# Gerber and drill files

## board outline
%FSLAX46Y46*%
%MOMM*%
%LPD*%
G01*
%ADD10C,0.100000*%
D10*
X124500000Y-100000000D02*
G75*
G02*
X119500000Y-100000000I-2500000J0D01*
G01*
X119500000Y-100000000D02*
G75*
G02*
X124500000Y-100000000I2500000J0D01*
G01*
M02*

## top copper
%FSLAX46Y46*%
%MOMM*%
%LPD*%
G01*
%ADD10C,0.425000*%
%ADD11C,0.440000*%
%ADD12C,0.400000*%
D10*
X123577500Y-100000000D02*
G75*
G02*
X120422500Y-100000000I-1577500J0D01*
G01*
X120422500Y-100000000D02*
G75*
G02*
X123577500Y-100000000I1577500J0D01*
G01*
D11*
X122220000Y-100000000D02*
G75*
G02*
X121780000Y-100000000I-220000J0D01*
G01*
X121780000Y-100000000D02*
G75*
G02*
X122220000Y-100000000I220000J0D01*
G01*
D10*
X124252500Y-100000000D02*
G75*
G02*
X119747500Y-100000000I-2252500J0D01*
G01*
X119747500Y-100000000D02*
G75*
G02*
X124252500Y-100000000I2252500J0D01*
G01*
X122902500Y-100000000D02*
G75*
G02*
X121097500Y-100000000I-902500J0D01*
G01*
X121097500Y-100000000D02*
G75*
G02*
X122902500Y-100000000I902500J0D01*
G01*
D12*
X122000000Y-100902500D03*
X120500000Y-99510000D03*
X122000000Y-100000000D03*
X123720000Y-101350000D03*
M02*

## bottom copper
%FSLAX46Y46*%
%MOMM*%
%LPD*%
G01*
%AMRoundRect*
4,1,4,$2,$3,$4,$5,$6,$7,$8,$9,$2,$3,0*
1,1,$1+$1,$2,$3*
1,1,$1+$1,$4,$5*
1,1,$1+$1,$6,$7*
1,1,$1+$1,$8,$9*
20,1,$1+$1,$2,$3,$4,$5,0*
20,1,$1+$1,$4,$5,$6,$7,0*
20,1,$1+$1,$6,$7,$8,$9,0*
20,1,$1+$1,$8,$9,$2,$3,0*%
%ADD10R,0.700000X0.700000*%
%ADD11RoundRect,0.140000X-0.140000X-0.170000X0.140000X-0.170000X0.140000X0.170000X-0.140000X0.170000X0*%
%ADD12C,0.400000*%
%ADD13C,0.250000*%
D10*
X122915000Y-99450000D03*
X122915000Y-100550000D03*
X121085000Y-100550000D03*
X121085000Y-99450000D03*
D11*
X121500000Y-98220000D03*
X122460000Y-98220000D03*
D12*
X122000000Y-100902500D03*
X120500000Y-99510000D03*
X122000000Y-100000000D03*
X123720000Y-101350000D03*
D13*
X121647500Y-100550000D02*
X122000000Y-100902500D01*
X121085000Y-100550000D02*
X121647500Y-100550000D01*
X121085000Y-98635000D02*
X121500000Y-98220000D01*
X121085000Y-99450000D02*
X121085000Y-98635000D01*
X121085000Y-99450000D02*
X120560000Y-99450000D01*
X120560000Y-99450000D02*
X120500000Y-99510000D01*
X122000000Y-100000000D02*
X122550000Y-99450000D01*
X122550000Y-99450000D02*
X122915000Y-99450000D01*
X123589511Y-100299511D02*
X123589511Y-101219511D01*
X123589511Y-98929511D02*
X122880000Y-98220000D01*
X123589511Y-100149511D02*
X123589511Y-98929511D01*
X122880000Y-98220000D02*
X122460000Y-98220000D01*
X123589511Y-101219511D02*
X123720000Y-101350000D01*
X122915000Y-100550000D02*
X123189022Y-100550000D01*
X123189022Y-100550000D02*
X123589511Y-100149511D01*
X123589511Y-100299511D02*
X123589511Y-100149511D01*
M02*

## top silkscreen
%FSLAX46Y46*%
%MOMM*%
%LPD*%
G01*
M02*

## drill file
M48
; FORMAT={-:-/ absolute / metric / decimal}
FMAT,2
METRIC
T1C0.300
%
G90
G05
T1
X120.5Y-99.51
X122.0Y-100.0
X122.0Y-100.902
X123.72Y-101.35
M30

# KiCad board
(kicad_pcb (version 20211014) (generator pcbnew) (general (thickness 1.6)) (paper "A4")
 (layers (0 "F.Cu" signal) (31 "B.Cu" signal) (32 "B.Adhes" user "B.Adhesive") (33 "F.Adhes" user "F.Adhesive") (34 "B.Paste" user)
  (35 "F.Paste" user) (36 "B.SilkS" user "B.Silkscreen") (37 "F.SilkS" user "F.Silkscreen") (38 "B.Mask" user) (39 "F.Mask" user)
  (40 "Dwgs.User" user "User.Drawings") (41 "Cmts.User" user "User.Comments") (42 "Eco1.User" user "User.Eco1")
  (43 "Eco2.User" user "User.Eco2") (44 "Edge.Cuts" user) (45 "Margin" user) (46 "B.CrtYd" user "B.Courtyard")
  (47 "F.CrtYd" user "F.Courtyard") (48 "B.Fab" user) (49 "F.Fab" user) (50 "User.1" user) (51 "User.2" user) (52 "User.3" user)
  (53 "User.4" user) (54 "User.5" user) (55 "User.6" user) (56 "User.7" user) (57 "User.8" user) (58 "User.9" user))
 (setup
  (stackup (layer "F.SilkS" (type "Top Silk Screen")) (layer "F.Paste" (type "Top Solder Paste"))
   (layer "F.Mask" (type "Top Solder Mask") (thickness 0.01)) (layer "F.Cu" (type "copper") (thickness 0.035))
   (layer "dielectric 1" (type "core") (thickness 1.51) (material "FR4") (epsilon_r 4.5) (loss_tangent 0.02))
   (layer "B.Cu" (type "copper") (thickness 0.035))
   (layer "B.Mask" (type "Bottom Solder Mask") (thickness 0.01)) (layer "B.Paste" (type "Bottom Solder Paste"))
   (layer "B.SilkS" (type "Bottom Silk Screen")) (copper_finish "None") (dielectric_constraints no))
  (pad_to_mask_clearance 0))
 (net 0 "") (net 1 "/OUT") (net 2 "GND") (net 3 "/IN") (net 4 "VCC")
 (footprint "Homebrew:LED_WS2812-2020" (layer "B.Cu") (at 122 100 180)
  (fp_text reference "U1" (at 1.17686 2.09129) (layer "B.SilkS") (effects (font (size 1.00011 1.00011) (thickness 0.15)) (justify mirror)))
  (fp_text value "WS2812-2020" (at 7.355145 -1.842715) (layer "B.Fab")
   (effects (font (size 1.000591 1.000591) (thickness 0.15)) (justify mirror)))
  (pad "1" smd rect (at -0.915 0.55 180) (size 0.7 0.7) (layers "B.Cu" "B.Paste" "B.Mask") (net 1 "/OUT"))
  (pad "2" smd rect (at -0.915 -0.55 180) (size 0.7 0.7) (layers "B.Cu" "B.Paste" "B.Mask") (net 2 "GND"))
  (pad "3" smd rect (at 0.915 -0.55) (size 0.7 0.7) (layers "B.Cu" "B.Paste" "B.Mask") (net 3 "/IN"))
  (pad "4" smd rect (at 0.915 0.55) (size 0.7 0.7) (layers "B.Cu" "B.Paste" "B.Mask") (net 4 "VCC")))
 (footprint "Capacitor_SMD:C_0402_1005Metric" (layer "B.Cu") (at 121.98 98.22)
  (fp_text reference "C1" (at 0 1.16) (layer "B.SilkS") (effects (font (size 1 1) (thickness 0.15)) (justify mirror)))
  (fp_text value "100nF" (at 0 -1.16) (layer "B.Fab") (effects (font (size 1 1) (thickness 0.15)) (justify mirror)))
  (pad "1" smd roundrect (at -0.48 0) (size 0.56 0.62) (layers "B.Cu" "B.Paste" "B.Mask") (roundrect_rratio 0.25) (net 4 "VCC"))
  (pad "2" smd roundrect (at 0.48 0) (size 0.56 0.62) (layers "B.Cu" "B.Paste" "B.Mask") (roundrect_rratio 0.25) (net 2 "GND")))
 (gr_circle (center 122 100) (end 123.5775 100) (layer "F.Cu") (width 0.425) (fill none))
 (gr_circle (center 122 100) (end 122.39 100) (layer "F.Cu") (width 0.1) (fill solid))
 (gr_circle (center 122 100) (end 124.2525 100) (layer "F.Cu") (width 0.425) (fill none))
 (gr_circle (center 122 100) (end 122.9025 100) (layer "F.Cu") (width 0.425) (fill none))
 (gr_circle (center 122 100) (end 124.5 100) (layer "Edge.Cuts") (width 0.1) (fill none))
 (via (at 122 100.9025) (size 0.4) (drill 0.3) (layers "F.Cu" "B.Cu") (free) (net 3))
 (segment (start 121.6475 100.55) (end 122 100.9025) (width 0.25) (layer "B.Cu") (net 3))
 (segment (start 121.085 100.55) (end 121.6475 100.55) (width 0.25) (layer "B.Cu") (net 3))
 (via (at 120.5 99.51) (size 0.4) (drill 0.3) (layers "F.Cu" "B.Cu") (free) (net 4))
 (segment (start 121.085 98.635) (end 121.5 98.22) (width 0.25) (layer "B.Cu") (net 4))
 (segment (start 121.085 99.45) (end 121.085 98.635) (width 0.25) (layer "B.Cu") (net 4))
 (segment (start 121.085 99.45) (end 120.56 99.45) (width 0.25) (layer "B.Cu") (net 4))
 (segment (start 120.56 99.45) (end 120.5 99.51) (width 0.25) (layer "B.Cu") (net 4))
 (via (at 122 100) (size 0.4) (drill 0.3) (layers "F.Cu" "B.Cu") (free) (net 1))
 (segment (start 122 100) (end 122.55 99.45) (width 0.25) (layer "B.Cu") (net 1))
 (segment (start 122.55 99.45) (end 122.915 99.45) (width 0.25) (layer "B.Cu") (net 1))
 (via (at 123.72 101.35) (size 0.4) (drill 0.3) (layers "F.Cu" "B.Cu") (free) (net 2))
 (segment (start 123.589511 100.299511) (end 123.589511 101.219511) (width 0.25) (layer "B.Cu") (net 2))
 (segment (start 123.589511 98.929511) (end 122.88 98.22) (width 0.25) (layer "B.Cu") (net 2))
 (segment (start 123.589511 100.149511) (end 123.589511 98.929511) (width 0.25) (layer "B.Cu") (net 2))
 (segment (start 122.88 98.22) (end 122.46 98.22) (width 0.25) (layer "B.Cu") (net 2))
 (segment (start 123.589511 101.219511) (end 123.72 101.35) (width 0.25) (layer "B.Cu") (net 2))
 (segment (start 122.915 100.55) (end 123.189022 100.55) (width 0.25) (layer "B.Cu") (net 2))
 (segment (start 123.189022 100.55) (end 123.589511 100.149511) (width 0.25) (layer "B.Cu") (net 2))
 (segment (start 123.589511 100.299511) (end 123.589511 100.149511) (width 0.25) (layer "B.Cu") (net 2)))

